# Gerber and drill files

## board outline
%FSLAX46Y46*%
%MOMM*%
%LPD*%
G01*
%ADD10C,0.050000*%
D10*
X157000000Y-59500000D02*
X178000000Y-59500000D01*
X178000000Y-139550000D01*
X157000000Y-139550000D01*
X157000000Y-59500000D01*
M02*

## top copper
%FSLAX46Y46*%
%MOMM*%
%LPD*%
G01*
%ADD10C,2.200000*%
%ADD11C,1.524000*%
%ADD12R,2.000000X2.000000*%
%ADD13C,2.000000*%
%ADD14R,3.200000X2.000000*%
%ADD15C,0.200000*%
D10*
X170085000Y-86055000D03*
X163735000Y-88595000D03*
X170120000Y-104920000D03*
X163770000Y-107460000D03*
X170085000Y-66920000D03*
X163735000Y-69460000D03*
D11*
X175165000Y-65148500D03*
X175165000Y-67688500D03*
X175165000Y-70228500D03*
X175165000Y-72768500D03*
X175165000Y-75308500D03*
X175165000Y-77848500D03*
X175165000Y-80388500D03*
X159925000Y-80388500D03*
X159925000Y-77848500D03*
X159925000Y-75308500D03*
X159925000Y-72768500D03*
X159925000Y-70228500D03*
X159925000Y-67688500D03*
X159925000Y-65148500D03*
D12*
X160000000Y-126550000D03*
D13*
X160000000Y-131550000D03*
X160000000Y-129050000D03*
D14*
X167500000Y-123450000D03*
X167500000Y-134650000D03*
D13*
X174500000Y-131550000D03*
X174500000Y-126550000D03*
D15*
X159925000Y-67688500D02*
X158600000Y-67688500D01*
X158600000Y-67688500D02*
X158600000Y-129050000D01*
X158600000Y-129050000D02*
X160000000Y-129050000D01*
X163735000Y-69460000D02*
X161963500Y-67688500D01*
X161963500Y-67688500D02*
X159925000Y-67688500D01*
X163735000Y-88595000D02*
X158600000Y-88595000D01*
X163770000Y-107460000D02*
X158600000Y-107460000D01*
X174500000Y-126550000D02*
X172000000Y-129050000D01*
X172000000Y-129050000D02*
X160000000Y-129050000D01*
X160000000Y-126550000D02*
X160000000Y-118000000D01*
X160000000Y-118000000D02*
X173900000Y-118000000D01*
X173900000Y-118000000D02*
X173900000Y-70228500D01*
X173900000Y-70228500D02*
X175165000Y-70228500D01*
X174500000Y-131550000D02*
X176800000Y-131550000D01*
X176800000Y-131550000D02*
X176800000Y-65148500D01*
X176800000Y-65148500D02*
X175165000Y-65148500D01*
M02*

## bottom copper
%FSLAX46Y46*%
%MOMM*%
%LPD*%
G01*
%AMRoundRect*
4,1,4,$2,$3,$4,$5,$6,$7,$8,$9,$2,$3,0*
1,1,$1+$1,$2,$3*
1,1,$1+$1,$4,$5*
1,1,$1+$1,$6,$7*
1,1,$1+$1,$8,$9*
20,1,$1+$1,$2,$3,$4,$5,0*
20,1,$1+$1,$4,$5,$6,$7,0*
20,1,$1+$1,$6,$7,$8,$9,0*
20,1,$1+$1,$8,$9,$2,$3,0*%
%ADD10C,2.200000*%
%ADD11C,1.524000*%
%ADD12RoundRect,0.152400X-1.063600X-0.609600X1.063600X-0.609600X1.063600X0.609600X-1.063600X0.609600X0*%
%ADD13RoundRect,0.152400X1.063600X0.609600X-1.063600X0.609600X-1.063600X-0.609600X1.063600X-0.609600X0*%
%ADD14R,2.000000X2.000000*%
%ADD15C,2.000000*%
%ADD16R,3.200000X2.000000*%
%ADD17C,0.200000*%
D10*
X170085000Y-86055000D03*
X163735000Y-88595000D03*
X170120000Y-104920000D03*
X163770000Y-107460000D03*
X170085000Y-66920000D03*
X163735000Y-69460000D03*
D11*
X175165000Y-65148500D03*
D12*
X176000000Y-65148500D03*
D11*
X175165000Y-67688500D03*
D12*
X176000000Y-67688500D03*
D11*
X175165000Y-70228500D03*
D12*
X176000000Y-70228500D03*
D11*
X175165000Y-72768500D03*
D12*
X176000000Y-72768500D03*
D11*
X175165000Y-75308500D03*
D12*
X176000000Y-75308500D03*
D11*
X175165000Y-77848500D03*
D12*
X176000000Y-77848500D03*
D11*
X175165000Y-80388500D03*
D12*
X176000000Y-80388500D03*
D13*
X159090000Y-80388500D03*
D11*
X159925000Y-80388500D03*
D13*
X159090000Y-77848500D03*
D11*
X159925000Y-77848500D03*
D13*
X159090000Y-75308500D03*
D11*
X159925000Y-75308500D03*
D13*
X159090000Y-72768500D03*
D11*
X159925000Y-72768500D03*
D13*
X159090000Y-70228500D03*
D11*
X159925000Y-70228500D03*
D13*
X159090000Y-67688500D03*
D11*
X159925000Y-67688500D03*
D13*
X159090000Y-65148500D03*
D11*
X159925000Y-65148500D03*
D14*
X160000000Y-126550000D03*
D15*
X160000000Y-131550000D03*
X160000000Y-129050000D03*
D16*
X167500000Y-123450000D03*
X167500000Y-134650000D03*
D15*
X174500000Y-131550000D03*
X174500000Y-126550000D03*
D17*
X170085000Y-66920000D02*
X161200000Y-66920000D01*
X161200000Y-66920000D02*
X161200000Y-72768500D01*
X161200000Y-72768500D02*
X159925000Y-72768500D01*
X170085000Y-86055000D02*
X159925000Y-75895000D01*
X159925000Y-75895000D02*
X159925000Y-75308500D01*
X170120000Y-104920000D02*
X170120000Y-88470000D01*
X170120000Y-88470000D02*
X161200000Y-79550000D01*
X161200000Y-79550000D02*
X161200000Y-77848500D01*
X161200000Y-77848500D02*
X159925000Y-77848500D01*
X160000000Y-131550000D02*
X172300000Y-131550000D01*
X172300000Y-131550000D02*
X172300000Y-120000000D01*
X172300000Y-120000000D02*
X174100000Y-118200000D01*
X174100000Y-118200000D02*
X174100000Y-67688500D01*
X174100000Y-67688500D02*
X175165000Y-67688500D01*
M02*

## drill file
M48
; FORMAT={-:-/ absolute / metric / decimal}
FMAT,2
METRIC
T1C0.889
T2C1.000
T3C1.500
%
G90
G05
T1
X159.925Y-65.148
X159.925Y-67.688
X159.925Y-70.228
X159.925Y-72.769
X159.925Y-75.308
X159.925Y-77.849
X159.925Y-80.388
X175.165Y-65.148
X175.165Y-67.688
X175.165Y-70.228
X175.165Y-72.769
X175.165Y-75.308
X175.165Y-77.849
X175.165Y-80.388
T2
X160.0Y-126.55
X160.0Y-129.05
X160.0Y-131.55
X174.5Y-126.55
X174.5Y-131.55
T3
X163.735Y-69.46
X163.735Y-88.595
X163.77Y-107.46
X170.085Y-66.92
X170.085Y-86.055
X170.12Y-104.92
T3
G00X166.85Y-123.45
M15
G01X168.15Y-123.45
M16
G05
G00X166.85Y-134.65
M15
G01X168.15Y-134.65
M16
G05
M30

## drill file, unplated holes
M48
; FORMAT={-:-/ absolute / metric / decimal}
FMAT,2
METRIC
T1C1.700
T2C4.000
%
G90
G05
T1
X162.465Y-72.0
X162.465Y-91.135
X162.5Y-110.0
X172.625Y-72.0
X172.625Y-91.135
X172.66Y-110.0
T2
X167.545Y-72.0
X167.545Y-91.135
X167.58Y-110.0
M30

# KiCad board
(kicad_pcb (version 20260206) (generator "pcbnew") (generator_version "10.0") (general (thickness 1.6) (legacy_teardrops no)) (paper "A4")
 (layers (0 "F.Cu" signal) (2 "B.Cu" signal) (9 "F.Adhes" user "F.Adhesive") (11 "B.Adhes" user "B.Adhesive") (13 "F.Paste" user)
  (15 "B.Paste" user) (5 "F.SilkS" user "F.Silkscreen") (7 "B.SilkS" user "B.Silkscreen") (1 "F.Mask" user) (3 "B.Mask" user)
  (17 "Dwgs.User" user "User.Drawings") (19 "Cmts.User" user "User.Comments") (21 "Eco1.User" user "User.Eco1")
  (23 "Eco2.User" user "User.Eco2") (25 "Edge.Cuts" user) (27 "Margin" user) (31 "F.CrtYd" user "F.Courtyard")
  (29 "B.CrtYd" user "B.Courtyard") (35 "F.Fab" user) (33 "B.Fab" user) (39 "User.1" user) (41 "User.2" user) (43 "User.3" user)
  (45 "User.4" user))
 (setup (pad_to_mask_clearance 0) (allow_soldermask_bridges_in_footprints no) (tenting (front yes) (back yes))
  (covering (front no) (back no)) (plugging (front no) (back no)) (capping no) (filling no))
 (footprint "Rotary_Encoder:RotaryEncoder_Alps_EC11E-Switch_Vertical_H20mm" (layer "F.Cu") (at 160 126.55)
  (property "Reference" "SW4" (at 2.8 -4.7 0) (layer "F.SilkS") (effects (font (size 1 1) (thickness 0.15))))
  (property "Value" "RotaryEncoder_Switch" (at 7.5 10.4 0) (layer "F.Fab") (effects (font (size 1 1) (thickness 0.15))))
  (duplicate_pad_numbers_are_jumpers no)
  (pad "A" thru_hole rect (at 0 0) (size 2 2) (drill 1) (layers "*.Cu" "*.Mask") (remove_unused_layers no) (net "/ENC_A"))
  (pad "B" thru_hole circle (at 0 5) (size 2 2) (drill 1) (layers "*.Cu" "*.Mask") (remove_unused_layers no) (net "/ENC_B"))
  (pad "C" thru_hole circle (at 0 2.5) (size 2 2) (drill 1) (layers "*.Cu" "*.Mask") (remove_unused_layers no) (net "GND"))
  (pad "MP" thru_hole rect (at 7.5 -3.1) (size 3.2 2) (drill oval 2.8 1.5) (layers "*.Cu" "*.Mask") (remove_unused_layers no))
  (pad "MP" thru_hole rect (at 7.5 8.1) (size 3.2 2) (drill oval 2.8 1.5) (layers "*.Cu" "*.Mask") (remove_unused_layers no))
  (pad "S1" thru_hole circle (at 14.5 5) (size 2 2) (drill 1) (layers "*.Cu" "*.Mask") (remove_unused_layers no) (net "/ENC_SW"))
  (pad "S2" thru_hole circle (at 14.5 0) (size 2 2) (drill 1) (layers "*.Cu" "*.Mask") (remove_unused_layers no) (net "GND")))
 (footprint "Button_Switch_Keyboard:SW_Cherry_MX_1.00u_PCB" (layer "F.Cu") (at 170.085 86.055)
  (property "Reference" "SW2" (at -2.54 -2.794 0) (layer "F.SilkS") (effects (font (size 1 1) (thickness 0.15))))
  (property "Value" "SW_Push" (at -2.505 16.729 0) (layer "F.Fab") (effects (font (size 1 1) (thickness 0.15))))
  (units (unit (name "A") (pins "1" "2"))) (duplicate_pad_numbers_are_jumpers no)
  (pad "" np_thru_hole circle (at -7.62 5.08) (size 1.7 1.7) (drill 1.7) (layers "*.Cu" "*.Mask"))
  (pad "" np_thru_hole circle (at -2.54 5.08) (size 4 4) (drill 4) (layers "*.Cu" "*.Mask"))
  (pad "" np_thru_hole circle (at 2.54 5.08) (size 1.7 1.7) (drill 1.7) (layers "*.Cu" "*.Mask"))
  (pad "1" thru_hole circle (at 0 0) (size 2.2 2.2) (drill 1.5) (layers "*.Cu" "*.Mask") (remove_unused_layers no)
   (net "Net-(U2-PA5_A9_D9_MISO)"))
  (pad "2" thru_hole circle (at -6.35 2.54) (size 2.2 2.2) (drill 1.5) (layers "*.Cu" "*.Mask") (remove_unused_layers no) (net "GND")))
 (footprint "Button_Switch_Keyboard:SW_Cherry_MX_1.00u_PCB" (layer "F.Cu") (at 170.12 104.92)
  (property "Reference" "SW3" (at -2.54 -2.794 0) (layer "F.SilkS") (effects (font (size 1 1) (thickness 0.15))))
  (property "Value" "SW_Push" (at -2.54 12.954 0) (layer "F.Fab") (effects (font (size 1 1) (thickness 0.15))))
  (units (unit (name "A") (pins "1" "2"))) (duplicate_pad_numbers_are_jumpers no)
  (pad "" np_thru_hole circle (at -7.62 5.08) (size 1.7 1.7) (drill 1.7) (layers "*.Cu" "*.Mask"))
  (pad "" np_thru_hole circle (at -2.54 5.08) (size 4 4) (drill 4) (layers "*.Cu" "*.Mask"))
  (pad "" np_thru_hole circle (at 2.54 5.08) (size 1.7 1.7) (drill 1.7) (layers "*.Cu" "*.Mask"))
  (pad "1" thru_hole circle (at 0 0) (size 2.2 2.2) (drill 1.5) (layers "*.Cu" "*.Mask") (remove_unused_layers no)
   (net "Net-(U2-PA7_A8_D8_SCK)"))
  (pad "2" thru_hole circle (at -6.35 2.54) (size 2.2 2.2) (drill 1.5) (layers "*.Cu" "*.Mask") (remove_unused_layers no) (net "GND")))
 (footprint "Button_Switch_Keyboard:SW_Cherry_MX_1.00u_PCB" (layer "F.Cu") (at 170.085 66.92)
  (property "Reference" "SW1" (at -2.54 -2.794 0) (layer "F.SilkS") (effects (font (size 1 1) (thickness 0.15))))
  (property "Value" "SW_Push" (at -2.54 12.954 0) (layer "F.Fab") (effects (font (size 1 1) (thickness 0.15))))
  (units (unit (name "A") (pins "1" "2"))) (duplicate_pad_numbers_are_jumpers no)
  (pad "" np_thru_hole circle (at -7.62 5.08) (size 1.7 1.7) (drill 1.7) (layers "*.Cu" "*.Mask"))
  (pad "" np_thru_hole circle (at -2.54 5.08) (size 4 4) (drill 4) (layers "*.Cu" "*.Mask"))
  (pad "" np_thru_hole circle (at 2.54 5.08) (size 1.7 1.7) (drill 1.7) (layers "*.Cu" "*.Mask"))
  (pad "1" thru_hole circle (at 0 0) (size 2.2 2.2) (drill 1.5) (layers "*.Cu" "*.Mask") (remove_unused_layers no)
   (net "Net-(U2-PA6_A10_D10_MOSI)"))
  (pad "2" thru_hole circle (at -6.35 2.54) (size 2.2 2.2) (drill 1.5) (layers "*.Cu" "*.Mask") (remove_unused_layers no) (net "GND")))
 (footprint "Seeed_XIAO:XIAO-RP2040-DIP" (layer "B.Cu") (at 167.545 72.7685 90)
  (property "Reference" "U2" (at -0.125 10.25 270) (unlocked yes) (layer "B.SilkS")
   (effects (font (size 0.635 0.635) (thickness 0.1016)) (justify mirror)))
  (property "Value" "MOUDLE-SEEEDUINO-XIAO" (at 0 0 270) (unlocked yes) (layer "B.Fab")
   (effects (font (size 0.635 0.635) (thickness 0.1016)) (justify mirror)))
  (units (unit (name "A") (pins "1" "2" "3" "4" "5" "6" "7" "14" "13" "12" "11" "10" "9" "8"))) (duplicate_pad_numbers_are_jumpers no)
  (pad "1" thru_hole circle (at 7.62 7.62) (size 1.524 1.524) (drill 0.889) (layers "*.Cu" "*.Mask") (remove_unused_layers no)
   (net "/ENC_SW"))
  (pad "1" smd roundrect (at 7.62 8.455) (size 2.432 1.524) (layers "B.Cu" "B.Mask") (roundrect_rratio 0.1) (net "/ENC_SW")
   (thermal_bridge_angle 45))
  (pad "2" thru_hole circle (at 5.08 7.62) (size 1.524 1.524) (drill 0.889) (layers "*.Cu" "*.Mask") (remove_unused_layers no)
   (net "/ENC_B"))
  (pad "2" smd roundrect (at 5.08 8.455) (size 2.432 1.524) (layers "B.Cu" "B.Mask") (roundrect_rratio 0.1) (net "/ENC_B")
   (thermal_bridge_angle 45))
  (pad "3" thru_hole circle (at 2.54 7.62) (size 1.524 1.524) (drill 0.889) (layers "*.Cu" "*.Mask") (remove_unused_layers no)
   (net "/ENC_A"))
  (pad "3" smd roundrect (at 2.54 8.455) (size 2.432 1.524) (layers "B.Cu" "B.Mask") (roundrect_rratio 0.1) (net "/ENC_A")
   (thermal_bridge_angle 45))
  (pad "4" thru_hole circle (at 0 7.62) (size 1.524 1.524) (drill 0.889) (layers "*.Cu" "*.Mask") (remove_unused_layers no)
   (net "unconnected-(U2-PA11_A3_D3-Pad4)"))
  (pad "4" smd roundrect (at 0 8.455) (size 2.432 1.524) (layers "B.Cu" "B.Mask") (roundrect_rratio 0.1)
   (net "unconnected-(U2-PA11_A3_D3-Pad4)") (thermal_bridge_angle 45))
  (pad "5" thru_hole circle (at -2.54 7.62) (size 1.524 1.524) (drill 0.889) (layers "*.Cu" "*.Mask") (remove_unused_layers no)
   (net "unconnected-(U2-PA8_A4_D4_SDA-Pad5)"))
  (pad "5" smd roundrect (at -2.54 8.455) (size 2.432 1.524) (layers "B.Cu" "B.Mask") (roundrect_rratio 0.1)
   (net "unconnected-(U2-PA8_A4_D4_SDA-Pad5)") (thermal_bridge_angle 45))
  (pad "6" thru_hole circle (at -5.08 7.62) (size 1.524 1.524) (drill 0.889) (layers "*.Cu" "*.Mask") (remove_unused_layers no)
   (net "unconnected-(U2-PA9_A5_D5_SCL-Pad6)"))
  (pad "6" smd roundrect (at -5.08 8.455) (size 2.432 1.524) (layers "B.Cu" "B.Mask") (roundrect_rratio 0.1)
   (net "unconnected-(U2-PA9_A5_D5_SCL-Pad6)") (thermal_bridge_angle 45))
  (pad "7" thru_hole circle (at -7.62 7.62) (size 1.524 1.524) (drill 0.889) (layers "*.Cu" "*.Mask") (remove_unused_layers no)
   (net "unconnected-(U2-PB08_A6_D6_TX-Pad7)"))
  (pad "7" smd roundrect (at -7.62 8.455) (size 2.432 1.524) (layers "B.Cu" "B.Mask") (roundrect_rratio 0.1)
   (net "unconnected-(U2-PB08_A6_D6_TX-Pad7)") (thermal_bridge_angle 45))
  (pad "8" smd roundrect (at -7.62 -8.455 180) (size 2.432 1.524) (layers "B.Cu" "B.Mask") (roundrect_rratio 0.1)
   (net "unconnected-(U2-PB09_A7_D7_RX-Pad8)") (thermal_bridge_angle 45))
  (pad "8" thru_hole circle (at -7.62 -7.62 180) (size 1.524 1.524) (drill 0.889) (layers "*.Cu" "*.Mask") (remove_unused_layers no)
   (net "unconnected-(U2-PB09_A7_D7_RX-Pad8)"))
  (pad "9" smd roundrect (at -5.08 -8.455 180) (size 2.432 1.524) (layers "B.Cu" "B.Mask") (roundrect_rratio 0.1)
   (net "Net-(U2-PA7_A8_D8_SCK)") (thermal_bridge_angle 45))
  (pad "9" thru_hole circle (at -5.08 -7.62 180) (size 1.524 1.524) (drill 0.889) (layers "*.Cu" "*.Mask") (remove_unused_layers no)
   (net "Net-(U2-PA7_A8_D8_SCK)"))
  (pad "10" smd roundrect (at -2.54 -8.455 180) (size 2.432 1.524) (layers "B.Cu" "B.Mask") (roundrect_rratio 0.1)
   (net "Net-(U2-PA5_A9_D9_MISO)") (thermal_bridge_angle 45))
  (pad "10" thru_hole circle (at -2.54 -7.62 180) (size 1.524 1.524) (drill 0.889) (layers "*.Cu" "*.Mask") (remove_unused_layers no)
   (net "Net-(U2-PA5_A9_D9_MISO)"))
  (pad "11" smd roundrect (at 0 -8.455 180) (size 2.432 1.524) (layers "B.Cu" "B.Mask") (roundrect_rratio 0.1)
   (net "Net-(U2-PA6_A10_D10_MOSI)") (thermal_bridge_angle 45))
  (pad "11" thru_hole circle (at 0 -7.62 180) (size 1.524 1.524) (drill 0.889) (layers "*.Cu" "*.Mask") (remove_unused_layers no)
   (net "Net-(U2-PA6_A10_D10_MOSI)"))
  (pad "12" smd roundrect (at 2.54 -8.455 180) (size 2.432 1.524) (layers "B.Cu" "B.Mask") (roundrect_rratio 0.1)
   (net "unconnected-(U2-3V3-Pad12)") (thermal_bridge_angle 45))
  (pad "12" thru_hole circle (at 2.54 -7.62 180) (size 1.524 1.524) (drill 0.889) (layers "*.Cu" "*.Mask") (remove_unused_layers no)
   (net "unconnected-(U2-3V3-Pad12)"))
  (pad "13" smd roundrect (at 5.08 -8.455 180) (size 2.432 1.524) (layers "B.Cu" "B.Mask") (roundrect_rratio 0.1) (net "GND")
   (thermal_bridge_angle 45))
  (pad "13" thru_hole circle (at 5.08 -7.62 180) (size 1.524 1.524) (drill 0.889) (layers "*.Cu" "*.Mask") (remove_unused_layers no)
   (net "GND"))
  (pad "14" smd roundrect (at 7.62 -8.455 180) (size 2.432 1.524) (layers "B.Cu" "B.Mask") (roundrect_rratio 0.1)
   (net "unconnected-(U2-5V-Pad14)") (thermal_bridge_angle 45))
  (pad "14" thru_hole circle (at 7.62 -7.62 180) (size 1.524 1.524) (drill 0.889) (layers "*.Cu" "*.Mask") (remove_unused_layers no)
   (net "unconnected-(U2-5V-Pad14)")))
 (gr_rect (start 157 59.5) (end 178 139.55) (stroke (width 0.05) (type default)) (fill no) (layer "Edge.Cuts"))
 (segment (start 159.925 75.895) (end 159.925 75.3085) (width 0.2) (layer "B.Cu") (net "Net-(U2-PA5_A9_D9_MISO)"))
 (segment (start 170.085 86.055) (end 159.925 75.895) (width 0.2) (layer "B.Cu") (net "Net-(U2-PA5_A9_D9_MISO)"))
 (segment (start 163.735 88.595) (end 158.6 88.595) (width 0.2) (layer "F.Cu") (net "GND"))
 (segment (start 163.77 107.46) (end 158.6 107.46) (width 0.2) (layer "F.Cu") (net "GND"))
 (segment (start 172 129.05) (end 160 129.05) (width 0.2) (layer "F.Cu") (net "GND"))
 (segment (start 158.6 67.6885) (end 158.6 129.05) (width 0.2) (layer "F.Cu") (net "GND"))
 (segment (start 174.5 126.55) (end 172 129.05) (width 0.2) (layer "F.Cu") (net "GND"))
 (segment (start 163.735 69.46) (end 161.9635 67.6885) (width 0.2) (layer "F.Cu") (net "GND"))
 (segment (start 158.6 129.05) (end 160 129.05) (width 0.2) (layer "F.Cu") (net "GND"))
 (segment (start 159.925 67.6885) (end 158.6 67.6885) (width 0.2) (layer "F.Cu") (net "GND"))
 (segment (start 161.9635 67.6885) (end 159.925 67.6885) (width 0.2) (layer "F.Cu") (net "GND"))
 (segment (start 170.12 104.92) (end 170.12 88.47) (width 0.2) (layer "B.Cu") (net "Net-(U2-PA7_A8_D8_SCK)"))
 (segment (start 161.2 77.8485) (end 159.925 77.8485) (width 0.2) (layer "B.Cu") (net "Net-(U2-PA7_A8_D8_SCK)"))
 (segment (start 161.2 79.55) (end 161.2 77.8485) (width 0.2) (layer "B.Cu") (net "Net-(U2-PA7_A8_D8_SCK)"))
 (segment (start 170.12 88.47) (end 161.2 79.55) (width 0.2) (layer "B.Cu") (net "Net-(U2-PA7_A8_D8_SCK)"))
 (segment (start 170.085 66.92) (end 161.2 66.92) (width 0.2) (layer "B.Cu") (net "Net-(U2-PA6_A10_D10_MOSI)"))
 (segment (start 161.2 66.92) (end 161.2 72.7685) (width 0.2) (layer "B.Cu") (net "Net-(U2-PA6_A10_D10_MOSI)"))
 (segment (start 161.2 72.7685) (end 159.925 72.7685) (width 0.2) (layer "B.Cu") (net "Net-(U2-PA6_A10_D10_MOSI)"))
 (segment (start 174.5 131.55) (end 176.8 131.55) (width 0.2) (layer "F.Cu") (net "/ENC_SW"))
 (segment (start 176.8 131.55) (end 176.8 65.1485) (width 0.2) (layer "F.Cu") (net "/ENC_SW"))
 (segment (start 176.8 65.1485) (end 175.165 65.1485) (width 0.2) (layer "F.Cu") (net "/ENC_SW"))
 (segment (start 172.3 120) (end 174.1 118.2) (width 0.2) (layer "B.Cu") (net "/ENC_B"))
 (segment (start 160 131.55) (end 172.3 131.55) (width 0.2) (layer "B.Cu") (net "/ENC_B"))
 (segment (start 174.1 67.6885) (end 175.165 67.6885) (width 0.2) (layer "B.Cu") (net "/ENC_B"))
 (segment (start 172.3 131.55) (end 172.3 120) (width 0.2) (layer "B.Cu") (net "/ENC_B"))
 (segment (start 174.1 118.2) (end 174.1 67.6885) (width 0.2) (layer "B.Cu") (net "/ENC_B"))
 (segment (start 173.9 118) (end 173.9 70.2285) (width 0.2) (layer "F.Cu") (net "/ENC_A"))
 (segment (start 160 126.55) (end 160 118) (width 0.2) (layer "F.Cu") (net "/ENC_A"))
 (segment (start 160 118) (end 173.9 118) (width 0.2) (layer "F.Cu") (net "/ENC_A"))
 (segment (start 173.9 70.2285) (end 175.165 70.2285) (width 0.2) (layer "F.Cu") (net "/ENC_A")))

